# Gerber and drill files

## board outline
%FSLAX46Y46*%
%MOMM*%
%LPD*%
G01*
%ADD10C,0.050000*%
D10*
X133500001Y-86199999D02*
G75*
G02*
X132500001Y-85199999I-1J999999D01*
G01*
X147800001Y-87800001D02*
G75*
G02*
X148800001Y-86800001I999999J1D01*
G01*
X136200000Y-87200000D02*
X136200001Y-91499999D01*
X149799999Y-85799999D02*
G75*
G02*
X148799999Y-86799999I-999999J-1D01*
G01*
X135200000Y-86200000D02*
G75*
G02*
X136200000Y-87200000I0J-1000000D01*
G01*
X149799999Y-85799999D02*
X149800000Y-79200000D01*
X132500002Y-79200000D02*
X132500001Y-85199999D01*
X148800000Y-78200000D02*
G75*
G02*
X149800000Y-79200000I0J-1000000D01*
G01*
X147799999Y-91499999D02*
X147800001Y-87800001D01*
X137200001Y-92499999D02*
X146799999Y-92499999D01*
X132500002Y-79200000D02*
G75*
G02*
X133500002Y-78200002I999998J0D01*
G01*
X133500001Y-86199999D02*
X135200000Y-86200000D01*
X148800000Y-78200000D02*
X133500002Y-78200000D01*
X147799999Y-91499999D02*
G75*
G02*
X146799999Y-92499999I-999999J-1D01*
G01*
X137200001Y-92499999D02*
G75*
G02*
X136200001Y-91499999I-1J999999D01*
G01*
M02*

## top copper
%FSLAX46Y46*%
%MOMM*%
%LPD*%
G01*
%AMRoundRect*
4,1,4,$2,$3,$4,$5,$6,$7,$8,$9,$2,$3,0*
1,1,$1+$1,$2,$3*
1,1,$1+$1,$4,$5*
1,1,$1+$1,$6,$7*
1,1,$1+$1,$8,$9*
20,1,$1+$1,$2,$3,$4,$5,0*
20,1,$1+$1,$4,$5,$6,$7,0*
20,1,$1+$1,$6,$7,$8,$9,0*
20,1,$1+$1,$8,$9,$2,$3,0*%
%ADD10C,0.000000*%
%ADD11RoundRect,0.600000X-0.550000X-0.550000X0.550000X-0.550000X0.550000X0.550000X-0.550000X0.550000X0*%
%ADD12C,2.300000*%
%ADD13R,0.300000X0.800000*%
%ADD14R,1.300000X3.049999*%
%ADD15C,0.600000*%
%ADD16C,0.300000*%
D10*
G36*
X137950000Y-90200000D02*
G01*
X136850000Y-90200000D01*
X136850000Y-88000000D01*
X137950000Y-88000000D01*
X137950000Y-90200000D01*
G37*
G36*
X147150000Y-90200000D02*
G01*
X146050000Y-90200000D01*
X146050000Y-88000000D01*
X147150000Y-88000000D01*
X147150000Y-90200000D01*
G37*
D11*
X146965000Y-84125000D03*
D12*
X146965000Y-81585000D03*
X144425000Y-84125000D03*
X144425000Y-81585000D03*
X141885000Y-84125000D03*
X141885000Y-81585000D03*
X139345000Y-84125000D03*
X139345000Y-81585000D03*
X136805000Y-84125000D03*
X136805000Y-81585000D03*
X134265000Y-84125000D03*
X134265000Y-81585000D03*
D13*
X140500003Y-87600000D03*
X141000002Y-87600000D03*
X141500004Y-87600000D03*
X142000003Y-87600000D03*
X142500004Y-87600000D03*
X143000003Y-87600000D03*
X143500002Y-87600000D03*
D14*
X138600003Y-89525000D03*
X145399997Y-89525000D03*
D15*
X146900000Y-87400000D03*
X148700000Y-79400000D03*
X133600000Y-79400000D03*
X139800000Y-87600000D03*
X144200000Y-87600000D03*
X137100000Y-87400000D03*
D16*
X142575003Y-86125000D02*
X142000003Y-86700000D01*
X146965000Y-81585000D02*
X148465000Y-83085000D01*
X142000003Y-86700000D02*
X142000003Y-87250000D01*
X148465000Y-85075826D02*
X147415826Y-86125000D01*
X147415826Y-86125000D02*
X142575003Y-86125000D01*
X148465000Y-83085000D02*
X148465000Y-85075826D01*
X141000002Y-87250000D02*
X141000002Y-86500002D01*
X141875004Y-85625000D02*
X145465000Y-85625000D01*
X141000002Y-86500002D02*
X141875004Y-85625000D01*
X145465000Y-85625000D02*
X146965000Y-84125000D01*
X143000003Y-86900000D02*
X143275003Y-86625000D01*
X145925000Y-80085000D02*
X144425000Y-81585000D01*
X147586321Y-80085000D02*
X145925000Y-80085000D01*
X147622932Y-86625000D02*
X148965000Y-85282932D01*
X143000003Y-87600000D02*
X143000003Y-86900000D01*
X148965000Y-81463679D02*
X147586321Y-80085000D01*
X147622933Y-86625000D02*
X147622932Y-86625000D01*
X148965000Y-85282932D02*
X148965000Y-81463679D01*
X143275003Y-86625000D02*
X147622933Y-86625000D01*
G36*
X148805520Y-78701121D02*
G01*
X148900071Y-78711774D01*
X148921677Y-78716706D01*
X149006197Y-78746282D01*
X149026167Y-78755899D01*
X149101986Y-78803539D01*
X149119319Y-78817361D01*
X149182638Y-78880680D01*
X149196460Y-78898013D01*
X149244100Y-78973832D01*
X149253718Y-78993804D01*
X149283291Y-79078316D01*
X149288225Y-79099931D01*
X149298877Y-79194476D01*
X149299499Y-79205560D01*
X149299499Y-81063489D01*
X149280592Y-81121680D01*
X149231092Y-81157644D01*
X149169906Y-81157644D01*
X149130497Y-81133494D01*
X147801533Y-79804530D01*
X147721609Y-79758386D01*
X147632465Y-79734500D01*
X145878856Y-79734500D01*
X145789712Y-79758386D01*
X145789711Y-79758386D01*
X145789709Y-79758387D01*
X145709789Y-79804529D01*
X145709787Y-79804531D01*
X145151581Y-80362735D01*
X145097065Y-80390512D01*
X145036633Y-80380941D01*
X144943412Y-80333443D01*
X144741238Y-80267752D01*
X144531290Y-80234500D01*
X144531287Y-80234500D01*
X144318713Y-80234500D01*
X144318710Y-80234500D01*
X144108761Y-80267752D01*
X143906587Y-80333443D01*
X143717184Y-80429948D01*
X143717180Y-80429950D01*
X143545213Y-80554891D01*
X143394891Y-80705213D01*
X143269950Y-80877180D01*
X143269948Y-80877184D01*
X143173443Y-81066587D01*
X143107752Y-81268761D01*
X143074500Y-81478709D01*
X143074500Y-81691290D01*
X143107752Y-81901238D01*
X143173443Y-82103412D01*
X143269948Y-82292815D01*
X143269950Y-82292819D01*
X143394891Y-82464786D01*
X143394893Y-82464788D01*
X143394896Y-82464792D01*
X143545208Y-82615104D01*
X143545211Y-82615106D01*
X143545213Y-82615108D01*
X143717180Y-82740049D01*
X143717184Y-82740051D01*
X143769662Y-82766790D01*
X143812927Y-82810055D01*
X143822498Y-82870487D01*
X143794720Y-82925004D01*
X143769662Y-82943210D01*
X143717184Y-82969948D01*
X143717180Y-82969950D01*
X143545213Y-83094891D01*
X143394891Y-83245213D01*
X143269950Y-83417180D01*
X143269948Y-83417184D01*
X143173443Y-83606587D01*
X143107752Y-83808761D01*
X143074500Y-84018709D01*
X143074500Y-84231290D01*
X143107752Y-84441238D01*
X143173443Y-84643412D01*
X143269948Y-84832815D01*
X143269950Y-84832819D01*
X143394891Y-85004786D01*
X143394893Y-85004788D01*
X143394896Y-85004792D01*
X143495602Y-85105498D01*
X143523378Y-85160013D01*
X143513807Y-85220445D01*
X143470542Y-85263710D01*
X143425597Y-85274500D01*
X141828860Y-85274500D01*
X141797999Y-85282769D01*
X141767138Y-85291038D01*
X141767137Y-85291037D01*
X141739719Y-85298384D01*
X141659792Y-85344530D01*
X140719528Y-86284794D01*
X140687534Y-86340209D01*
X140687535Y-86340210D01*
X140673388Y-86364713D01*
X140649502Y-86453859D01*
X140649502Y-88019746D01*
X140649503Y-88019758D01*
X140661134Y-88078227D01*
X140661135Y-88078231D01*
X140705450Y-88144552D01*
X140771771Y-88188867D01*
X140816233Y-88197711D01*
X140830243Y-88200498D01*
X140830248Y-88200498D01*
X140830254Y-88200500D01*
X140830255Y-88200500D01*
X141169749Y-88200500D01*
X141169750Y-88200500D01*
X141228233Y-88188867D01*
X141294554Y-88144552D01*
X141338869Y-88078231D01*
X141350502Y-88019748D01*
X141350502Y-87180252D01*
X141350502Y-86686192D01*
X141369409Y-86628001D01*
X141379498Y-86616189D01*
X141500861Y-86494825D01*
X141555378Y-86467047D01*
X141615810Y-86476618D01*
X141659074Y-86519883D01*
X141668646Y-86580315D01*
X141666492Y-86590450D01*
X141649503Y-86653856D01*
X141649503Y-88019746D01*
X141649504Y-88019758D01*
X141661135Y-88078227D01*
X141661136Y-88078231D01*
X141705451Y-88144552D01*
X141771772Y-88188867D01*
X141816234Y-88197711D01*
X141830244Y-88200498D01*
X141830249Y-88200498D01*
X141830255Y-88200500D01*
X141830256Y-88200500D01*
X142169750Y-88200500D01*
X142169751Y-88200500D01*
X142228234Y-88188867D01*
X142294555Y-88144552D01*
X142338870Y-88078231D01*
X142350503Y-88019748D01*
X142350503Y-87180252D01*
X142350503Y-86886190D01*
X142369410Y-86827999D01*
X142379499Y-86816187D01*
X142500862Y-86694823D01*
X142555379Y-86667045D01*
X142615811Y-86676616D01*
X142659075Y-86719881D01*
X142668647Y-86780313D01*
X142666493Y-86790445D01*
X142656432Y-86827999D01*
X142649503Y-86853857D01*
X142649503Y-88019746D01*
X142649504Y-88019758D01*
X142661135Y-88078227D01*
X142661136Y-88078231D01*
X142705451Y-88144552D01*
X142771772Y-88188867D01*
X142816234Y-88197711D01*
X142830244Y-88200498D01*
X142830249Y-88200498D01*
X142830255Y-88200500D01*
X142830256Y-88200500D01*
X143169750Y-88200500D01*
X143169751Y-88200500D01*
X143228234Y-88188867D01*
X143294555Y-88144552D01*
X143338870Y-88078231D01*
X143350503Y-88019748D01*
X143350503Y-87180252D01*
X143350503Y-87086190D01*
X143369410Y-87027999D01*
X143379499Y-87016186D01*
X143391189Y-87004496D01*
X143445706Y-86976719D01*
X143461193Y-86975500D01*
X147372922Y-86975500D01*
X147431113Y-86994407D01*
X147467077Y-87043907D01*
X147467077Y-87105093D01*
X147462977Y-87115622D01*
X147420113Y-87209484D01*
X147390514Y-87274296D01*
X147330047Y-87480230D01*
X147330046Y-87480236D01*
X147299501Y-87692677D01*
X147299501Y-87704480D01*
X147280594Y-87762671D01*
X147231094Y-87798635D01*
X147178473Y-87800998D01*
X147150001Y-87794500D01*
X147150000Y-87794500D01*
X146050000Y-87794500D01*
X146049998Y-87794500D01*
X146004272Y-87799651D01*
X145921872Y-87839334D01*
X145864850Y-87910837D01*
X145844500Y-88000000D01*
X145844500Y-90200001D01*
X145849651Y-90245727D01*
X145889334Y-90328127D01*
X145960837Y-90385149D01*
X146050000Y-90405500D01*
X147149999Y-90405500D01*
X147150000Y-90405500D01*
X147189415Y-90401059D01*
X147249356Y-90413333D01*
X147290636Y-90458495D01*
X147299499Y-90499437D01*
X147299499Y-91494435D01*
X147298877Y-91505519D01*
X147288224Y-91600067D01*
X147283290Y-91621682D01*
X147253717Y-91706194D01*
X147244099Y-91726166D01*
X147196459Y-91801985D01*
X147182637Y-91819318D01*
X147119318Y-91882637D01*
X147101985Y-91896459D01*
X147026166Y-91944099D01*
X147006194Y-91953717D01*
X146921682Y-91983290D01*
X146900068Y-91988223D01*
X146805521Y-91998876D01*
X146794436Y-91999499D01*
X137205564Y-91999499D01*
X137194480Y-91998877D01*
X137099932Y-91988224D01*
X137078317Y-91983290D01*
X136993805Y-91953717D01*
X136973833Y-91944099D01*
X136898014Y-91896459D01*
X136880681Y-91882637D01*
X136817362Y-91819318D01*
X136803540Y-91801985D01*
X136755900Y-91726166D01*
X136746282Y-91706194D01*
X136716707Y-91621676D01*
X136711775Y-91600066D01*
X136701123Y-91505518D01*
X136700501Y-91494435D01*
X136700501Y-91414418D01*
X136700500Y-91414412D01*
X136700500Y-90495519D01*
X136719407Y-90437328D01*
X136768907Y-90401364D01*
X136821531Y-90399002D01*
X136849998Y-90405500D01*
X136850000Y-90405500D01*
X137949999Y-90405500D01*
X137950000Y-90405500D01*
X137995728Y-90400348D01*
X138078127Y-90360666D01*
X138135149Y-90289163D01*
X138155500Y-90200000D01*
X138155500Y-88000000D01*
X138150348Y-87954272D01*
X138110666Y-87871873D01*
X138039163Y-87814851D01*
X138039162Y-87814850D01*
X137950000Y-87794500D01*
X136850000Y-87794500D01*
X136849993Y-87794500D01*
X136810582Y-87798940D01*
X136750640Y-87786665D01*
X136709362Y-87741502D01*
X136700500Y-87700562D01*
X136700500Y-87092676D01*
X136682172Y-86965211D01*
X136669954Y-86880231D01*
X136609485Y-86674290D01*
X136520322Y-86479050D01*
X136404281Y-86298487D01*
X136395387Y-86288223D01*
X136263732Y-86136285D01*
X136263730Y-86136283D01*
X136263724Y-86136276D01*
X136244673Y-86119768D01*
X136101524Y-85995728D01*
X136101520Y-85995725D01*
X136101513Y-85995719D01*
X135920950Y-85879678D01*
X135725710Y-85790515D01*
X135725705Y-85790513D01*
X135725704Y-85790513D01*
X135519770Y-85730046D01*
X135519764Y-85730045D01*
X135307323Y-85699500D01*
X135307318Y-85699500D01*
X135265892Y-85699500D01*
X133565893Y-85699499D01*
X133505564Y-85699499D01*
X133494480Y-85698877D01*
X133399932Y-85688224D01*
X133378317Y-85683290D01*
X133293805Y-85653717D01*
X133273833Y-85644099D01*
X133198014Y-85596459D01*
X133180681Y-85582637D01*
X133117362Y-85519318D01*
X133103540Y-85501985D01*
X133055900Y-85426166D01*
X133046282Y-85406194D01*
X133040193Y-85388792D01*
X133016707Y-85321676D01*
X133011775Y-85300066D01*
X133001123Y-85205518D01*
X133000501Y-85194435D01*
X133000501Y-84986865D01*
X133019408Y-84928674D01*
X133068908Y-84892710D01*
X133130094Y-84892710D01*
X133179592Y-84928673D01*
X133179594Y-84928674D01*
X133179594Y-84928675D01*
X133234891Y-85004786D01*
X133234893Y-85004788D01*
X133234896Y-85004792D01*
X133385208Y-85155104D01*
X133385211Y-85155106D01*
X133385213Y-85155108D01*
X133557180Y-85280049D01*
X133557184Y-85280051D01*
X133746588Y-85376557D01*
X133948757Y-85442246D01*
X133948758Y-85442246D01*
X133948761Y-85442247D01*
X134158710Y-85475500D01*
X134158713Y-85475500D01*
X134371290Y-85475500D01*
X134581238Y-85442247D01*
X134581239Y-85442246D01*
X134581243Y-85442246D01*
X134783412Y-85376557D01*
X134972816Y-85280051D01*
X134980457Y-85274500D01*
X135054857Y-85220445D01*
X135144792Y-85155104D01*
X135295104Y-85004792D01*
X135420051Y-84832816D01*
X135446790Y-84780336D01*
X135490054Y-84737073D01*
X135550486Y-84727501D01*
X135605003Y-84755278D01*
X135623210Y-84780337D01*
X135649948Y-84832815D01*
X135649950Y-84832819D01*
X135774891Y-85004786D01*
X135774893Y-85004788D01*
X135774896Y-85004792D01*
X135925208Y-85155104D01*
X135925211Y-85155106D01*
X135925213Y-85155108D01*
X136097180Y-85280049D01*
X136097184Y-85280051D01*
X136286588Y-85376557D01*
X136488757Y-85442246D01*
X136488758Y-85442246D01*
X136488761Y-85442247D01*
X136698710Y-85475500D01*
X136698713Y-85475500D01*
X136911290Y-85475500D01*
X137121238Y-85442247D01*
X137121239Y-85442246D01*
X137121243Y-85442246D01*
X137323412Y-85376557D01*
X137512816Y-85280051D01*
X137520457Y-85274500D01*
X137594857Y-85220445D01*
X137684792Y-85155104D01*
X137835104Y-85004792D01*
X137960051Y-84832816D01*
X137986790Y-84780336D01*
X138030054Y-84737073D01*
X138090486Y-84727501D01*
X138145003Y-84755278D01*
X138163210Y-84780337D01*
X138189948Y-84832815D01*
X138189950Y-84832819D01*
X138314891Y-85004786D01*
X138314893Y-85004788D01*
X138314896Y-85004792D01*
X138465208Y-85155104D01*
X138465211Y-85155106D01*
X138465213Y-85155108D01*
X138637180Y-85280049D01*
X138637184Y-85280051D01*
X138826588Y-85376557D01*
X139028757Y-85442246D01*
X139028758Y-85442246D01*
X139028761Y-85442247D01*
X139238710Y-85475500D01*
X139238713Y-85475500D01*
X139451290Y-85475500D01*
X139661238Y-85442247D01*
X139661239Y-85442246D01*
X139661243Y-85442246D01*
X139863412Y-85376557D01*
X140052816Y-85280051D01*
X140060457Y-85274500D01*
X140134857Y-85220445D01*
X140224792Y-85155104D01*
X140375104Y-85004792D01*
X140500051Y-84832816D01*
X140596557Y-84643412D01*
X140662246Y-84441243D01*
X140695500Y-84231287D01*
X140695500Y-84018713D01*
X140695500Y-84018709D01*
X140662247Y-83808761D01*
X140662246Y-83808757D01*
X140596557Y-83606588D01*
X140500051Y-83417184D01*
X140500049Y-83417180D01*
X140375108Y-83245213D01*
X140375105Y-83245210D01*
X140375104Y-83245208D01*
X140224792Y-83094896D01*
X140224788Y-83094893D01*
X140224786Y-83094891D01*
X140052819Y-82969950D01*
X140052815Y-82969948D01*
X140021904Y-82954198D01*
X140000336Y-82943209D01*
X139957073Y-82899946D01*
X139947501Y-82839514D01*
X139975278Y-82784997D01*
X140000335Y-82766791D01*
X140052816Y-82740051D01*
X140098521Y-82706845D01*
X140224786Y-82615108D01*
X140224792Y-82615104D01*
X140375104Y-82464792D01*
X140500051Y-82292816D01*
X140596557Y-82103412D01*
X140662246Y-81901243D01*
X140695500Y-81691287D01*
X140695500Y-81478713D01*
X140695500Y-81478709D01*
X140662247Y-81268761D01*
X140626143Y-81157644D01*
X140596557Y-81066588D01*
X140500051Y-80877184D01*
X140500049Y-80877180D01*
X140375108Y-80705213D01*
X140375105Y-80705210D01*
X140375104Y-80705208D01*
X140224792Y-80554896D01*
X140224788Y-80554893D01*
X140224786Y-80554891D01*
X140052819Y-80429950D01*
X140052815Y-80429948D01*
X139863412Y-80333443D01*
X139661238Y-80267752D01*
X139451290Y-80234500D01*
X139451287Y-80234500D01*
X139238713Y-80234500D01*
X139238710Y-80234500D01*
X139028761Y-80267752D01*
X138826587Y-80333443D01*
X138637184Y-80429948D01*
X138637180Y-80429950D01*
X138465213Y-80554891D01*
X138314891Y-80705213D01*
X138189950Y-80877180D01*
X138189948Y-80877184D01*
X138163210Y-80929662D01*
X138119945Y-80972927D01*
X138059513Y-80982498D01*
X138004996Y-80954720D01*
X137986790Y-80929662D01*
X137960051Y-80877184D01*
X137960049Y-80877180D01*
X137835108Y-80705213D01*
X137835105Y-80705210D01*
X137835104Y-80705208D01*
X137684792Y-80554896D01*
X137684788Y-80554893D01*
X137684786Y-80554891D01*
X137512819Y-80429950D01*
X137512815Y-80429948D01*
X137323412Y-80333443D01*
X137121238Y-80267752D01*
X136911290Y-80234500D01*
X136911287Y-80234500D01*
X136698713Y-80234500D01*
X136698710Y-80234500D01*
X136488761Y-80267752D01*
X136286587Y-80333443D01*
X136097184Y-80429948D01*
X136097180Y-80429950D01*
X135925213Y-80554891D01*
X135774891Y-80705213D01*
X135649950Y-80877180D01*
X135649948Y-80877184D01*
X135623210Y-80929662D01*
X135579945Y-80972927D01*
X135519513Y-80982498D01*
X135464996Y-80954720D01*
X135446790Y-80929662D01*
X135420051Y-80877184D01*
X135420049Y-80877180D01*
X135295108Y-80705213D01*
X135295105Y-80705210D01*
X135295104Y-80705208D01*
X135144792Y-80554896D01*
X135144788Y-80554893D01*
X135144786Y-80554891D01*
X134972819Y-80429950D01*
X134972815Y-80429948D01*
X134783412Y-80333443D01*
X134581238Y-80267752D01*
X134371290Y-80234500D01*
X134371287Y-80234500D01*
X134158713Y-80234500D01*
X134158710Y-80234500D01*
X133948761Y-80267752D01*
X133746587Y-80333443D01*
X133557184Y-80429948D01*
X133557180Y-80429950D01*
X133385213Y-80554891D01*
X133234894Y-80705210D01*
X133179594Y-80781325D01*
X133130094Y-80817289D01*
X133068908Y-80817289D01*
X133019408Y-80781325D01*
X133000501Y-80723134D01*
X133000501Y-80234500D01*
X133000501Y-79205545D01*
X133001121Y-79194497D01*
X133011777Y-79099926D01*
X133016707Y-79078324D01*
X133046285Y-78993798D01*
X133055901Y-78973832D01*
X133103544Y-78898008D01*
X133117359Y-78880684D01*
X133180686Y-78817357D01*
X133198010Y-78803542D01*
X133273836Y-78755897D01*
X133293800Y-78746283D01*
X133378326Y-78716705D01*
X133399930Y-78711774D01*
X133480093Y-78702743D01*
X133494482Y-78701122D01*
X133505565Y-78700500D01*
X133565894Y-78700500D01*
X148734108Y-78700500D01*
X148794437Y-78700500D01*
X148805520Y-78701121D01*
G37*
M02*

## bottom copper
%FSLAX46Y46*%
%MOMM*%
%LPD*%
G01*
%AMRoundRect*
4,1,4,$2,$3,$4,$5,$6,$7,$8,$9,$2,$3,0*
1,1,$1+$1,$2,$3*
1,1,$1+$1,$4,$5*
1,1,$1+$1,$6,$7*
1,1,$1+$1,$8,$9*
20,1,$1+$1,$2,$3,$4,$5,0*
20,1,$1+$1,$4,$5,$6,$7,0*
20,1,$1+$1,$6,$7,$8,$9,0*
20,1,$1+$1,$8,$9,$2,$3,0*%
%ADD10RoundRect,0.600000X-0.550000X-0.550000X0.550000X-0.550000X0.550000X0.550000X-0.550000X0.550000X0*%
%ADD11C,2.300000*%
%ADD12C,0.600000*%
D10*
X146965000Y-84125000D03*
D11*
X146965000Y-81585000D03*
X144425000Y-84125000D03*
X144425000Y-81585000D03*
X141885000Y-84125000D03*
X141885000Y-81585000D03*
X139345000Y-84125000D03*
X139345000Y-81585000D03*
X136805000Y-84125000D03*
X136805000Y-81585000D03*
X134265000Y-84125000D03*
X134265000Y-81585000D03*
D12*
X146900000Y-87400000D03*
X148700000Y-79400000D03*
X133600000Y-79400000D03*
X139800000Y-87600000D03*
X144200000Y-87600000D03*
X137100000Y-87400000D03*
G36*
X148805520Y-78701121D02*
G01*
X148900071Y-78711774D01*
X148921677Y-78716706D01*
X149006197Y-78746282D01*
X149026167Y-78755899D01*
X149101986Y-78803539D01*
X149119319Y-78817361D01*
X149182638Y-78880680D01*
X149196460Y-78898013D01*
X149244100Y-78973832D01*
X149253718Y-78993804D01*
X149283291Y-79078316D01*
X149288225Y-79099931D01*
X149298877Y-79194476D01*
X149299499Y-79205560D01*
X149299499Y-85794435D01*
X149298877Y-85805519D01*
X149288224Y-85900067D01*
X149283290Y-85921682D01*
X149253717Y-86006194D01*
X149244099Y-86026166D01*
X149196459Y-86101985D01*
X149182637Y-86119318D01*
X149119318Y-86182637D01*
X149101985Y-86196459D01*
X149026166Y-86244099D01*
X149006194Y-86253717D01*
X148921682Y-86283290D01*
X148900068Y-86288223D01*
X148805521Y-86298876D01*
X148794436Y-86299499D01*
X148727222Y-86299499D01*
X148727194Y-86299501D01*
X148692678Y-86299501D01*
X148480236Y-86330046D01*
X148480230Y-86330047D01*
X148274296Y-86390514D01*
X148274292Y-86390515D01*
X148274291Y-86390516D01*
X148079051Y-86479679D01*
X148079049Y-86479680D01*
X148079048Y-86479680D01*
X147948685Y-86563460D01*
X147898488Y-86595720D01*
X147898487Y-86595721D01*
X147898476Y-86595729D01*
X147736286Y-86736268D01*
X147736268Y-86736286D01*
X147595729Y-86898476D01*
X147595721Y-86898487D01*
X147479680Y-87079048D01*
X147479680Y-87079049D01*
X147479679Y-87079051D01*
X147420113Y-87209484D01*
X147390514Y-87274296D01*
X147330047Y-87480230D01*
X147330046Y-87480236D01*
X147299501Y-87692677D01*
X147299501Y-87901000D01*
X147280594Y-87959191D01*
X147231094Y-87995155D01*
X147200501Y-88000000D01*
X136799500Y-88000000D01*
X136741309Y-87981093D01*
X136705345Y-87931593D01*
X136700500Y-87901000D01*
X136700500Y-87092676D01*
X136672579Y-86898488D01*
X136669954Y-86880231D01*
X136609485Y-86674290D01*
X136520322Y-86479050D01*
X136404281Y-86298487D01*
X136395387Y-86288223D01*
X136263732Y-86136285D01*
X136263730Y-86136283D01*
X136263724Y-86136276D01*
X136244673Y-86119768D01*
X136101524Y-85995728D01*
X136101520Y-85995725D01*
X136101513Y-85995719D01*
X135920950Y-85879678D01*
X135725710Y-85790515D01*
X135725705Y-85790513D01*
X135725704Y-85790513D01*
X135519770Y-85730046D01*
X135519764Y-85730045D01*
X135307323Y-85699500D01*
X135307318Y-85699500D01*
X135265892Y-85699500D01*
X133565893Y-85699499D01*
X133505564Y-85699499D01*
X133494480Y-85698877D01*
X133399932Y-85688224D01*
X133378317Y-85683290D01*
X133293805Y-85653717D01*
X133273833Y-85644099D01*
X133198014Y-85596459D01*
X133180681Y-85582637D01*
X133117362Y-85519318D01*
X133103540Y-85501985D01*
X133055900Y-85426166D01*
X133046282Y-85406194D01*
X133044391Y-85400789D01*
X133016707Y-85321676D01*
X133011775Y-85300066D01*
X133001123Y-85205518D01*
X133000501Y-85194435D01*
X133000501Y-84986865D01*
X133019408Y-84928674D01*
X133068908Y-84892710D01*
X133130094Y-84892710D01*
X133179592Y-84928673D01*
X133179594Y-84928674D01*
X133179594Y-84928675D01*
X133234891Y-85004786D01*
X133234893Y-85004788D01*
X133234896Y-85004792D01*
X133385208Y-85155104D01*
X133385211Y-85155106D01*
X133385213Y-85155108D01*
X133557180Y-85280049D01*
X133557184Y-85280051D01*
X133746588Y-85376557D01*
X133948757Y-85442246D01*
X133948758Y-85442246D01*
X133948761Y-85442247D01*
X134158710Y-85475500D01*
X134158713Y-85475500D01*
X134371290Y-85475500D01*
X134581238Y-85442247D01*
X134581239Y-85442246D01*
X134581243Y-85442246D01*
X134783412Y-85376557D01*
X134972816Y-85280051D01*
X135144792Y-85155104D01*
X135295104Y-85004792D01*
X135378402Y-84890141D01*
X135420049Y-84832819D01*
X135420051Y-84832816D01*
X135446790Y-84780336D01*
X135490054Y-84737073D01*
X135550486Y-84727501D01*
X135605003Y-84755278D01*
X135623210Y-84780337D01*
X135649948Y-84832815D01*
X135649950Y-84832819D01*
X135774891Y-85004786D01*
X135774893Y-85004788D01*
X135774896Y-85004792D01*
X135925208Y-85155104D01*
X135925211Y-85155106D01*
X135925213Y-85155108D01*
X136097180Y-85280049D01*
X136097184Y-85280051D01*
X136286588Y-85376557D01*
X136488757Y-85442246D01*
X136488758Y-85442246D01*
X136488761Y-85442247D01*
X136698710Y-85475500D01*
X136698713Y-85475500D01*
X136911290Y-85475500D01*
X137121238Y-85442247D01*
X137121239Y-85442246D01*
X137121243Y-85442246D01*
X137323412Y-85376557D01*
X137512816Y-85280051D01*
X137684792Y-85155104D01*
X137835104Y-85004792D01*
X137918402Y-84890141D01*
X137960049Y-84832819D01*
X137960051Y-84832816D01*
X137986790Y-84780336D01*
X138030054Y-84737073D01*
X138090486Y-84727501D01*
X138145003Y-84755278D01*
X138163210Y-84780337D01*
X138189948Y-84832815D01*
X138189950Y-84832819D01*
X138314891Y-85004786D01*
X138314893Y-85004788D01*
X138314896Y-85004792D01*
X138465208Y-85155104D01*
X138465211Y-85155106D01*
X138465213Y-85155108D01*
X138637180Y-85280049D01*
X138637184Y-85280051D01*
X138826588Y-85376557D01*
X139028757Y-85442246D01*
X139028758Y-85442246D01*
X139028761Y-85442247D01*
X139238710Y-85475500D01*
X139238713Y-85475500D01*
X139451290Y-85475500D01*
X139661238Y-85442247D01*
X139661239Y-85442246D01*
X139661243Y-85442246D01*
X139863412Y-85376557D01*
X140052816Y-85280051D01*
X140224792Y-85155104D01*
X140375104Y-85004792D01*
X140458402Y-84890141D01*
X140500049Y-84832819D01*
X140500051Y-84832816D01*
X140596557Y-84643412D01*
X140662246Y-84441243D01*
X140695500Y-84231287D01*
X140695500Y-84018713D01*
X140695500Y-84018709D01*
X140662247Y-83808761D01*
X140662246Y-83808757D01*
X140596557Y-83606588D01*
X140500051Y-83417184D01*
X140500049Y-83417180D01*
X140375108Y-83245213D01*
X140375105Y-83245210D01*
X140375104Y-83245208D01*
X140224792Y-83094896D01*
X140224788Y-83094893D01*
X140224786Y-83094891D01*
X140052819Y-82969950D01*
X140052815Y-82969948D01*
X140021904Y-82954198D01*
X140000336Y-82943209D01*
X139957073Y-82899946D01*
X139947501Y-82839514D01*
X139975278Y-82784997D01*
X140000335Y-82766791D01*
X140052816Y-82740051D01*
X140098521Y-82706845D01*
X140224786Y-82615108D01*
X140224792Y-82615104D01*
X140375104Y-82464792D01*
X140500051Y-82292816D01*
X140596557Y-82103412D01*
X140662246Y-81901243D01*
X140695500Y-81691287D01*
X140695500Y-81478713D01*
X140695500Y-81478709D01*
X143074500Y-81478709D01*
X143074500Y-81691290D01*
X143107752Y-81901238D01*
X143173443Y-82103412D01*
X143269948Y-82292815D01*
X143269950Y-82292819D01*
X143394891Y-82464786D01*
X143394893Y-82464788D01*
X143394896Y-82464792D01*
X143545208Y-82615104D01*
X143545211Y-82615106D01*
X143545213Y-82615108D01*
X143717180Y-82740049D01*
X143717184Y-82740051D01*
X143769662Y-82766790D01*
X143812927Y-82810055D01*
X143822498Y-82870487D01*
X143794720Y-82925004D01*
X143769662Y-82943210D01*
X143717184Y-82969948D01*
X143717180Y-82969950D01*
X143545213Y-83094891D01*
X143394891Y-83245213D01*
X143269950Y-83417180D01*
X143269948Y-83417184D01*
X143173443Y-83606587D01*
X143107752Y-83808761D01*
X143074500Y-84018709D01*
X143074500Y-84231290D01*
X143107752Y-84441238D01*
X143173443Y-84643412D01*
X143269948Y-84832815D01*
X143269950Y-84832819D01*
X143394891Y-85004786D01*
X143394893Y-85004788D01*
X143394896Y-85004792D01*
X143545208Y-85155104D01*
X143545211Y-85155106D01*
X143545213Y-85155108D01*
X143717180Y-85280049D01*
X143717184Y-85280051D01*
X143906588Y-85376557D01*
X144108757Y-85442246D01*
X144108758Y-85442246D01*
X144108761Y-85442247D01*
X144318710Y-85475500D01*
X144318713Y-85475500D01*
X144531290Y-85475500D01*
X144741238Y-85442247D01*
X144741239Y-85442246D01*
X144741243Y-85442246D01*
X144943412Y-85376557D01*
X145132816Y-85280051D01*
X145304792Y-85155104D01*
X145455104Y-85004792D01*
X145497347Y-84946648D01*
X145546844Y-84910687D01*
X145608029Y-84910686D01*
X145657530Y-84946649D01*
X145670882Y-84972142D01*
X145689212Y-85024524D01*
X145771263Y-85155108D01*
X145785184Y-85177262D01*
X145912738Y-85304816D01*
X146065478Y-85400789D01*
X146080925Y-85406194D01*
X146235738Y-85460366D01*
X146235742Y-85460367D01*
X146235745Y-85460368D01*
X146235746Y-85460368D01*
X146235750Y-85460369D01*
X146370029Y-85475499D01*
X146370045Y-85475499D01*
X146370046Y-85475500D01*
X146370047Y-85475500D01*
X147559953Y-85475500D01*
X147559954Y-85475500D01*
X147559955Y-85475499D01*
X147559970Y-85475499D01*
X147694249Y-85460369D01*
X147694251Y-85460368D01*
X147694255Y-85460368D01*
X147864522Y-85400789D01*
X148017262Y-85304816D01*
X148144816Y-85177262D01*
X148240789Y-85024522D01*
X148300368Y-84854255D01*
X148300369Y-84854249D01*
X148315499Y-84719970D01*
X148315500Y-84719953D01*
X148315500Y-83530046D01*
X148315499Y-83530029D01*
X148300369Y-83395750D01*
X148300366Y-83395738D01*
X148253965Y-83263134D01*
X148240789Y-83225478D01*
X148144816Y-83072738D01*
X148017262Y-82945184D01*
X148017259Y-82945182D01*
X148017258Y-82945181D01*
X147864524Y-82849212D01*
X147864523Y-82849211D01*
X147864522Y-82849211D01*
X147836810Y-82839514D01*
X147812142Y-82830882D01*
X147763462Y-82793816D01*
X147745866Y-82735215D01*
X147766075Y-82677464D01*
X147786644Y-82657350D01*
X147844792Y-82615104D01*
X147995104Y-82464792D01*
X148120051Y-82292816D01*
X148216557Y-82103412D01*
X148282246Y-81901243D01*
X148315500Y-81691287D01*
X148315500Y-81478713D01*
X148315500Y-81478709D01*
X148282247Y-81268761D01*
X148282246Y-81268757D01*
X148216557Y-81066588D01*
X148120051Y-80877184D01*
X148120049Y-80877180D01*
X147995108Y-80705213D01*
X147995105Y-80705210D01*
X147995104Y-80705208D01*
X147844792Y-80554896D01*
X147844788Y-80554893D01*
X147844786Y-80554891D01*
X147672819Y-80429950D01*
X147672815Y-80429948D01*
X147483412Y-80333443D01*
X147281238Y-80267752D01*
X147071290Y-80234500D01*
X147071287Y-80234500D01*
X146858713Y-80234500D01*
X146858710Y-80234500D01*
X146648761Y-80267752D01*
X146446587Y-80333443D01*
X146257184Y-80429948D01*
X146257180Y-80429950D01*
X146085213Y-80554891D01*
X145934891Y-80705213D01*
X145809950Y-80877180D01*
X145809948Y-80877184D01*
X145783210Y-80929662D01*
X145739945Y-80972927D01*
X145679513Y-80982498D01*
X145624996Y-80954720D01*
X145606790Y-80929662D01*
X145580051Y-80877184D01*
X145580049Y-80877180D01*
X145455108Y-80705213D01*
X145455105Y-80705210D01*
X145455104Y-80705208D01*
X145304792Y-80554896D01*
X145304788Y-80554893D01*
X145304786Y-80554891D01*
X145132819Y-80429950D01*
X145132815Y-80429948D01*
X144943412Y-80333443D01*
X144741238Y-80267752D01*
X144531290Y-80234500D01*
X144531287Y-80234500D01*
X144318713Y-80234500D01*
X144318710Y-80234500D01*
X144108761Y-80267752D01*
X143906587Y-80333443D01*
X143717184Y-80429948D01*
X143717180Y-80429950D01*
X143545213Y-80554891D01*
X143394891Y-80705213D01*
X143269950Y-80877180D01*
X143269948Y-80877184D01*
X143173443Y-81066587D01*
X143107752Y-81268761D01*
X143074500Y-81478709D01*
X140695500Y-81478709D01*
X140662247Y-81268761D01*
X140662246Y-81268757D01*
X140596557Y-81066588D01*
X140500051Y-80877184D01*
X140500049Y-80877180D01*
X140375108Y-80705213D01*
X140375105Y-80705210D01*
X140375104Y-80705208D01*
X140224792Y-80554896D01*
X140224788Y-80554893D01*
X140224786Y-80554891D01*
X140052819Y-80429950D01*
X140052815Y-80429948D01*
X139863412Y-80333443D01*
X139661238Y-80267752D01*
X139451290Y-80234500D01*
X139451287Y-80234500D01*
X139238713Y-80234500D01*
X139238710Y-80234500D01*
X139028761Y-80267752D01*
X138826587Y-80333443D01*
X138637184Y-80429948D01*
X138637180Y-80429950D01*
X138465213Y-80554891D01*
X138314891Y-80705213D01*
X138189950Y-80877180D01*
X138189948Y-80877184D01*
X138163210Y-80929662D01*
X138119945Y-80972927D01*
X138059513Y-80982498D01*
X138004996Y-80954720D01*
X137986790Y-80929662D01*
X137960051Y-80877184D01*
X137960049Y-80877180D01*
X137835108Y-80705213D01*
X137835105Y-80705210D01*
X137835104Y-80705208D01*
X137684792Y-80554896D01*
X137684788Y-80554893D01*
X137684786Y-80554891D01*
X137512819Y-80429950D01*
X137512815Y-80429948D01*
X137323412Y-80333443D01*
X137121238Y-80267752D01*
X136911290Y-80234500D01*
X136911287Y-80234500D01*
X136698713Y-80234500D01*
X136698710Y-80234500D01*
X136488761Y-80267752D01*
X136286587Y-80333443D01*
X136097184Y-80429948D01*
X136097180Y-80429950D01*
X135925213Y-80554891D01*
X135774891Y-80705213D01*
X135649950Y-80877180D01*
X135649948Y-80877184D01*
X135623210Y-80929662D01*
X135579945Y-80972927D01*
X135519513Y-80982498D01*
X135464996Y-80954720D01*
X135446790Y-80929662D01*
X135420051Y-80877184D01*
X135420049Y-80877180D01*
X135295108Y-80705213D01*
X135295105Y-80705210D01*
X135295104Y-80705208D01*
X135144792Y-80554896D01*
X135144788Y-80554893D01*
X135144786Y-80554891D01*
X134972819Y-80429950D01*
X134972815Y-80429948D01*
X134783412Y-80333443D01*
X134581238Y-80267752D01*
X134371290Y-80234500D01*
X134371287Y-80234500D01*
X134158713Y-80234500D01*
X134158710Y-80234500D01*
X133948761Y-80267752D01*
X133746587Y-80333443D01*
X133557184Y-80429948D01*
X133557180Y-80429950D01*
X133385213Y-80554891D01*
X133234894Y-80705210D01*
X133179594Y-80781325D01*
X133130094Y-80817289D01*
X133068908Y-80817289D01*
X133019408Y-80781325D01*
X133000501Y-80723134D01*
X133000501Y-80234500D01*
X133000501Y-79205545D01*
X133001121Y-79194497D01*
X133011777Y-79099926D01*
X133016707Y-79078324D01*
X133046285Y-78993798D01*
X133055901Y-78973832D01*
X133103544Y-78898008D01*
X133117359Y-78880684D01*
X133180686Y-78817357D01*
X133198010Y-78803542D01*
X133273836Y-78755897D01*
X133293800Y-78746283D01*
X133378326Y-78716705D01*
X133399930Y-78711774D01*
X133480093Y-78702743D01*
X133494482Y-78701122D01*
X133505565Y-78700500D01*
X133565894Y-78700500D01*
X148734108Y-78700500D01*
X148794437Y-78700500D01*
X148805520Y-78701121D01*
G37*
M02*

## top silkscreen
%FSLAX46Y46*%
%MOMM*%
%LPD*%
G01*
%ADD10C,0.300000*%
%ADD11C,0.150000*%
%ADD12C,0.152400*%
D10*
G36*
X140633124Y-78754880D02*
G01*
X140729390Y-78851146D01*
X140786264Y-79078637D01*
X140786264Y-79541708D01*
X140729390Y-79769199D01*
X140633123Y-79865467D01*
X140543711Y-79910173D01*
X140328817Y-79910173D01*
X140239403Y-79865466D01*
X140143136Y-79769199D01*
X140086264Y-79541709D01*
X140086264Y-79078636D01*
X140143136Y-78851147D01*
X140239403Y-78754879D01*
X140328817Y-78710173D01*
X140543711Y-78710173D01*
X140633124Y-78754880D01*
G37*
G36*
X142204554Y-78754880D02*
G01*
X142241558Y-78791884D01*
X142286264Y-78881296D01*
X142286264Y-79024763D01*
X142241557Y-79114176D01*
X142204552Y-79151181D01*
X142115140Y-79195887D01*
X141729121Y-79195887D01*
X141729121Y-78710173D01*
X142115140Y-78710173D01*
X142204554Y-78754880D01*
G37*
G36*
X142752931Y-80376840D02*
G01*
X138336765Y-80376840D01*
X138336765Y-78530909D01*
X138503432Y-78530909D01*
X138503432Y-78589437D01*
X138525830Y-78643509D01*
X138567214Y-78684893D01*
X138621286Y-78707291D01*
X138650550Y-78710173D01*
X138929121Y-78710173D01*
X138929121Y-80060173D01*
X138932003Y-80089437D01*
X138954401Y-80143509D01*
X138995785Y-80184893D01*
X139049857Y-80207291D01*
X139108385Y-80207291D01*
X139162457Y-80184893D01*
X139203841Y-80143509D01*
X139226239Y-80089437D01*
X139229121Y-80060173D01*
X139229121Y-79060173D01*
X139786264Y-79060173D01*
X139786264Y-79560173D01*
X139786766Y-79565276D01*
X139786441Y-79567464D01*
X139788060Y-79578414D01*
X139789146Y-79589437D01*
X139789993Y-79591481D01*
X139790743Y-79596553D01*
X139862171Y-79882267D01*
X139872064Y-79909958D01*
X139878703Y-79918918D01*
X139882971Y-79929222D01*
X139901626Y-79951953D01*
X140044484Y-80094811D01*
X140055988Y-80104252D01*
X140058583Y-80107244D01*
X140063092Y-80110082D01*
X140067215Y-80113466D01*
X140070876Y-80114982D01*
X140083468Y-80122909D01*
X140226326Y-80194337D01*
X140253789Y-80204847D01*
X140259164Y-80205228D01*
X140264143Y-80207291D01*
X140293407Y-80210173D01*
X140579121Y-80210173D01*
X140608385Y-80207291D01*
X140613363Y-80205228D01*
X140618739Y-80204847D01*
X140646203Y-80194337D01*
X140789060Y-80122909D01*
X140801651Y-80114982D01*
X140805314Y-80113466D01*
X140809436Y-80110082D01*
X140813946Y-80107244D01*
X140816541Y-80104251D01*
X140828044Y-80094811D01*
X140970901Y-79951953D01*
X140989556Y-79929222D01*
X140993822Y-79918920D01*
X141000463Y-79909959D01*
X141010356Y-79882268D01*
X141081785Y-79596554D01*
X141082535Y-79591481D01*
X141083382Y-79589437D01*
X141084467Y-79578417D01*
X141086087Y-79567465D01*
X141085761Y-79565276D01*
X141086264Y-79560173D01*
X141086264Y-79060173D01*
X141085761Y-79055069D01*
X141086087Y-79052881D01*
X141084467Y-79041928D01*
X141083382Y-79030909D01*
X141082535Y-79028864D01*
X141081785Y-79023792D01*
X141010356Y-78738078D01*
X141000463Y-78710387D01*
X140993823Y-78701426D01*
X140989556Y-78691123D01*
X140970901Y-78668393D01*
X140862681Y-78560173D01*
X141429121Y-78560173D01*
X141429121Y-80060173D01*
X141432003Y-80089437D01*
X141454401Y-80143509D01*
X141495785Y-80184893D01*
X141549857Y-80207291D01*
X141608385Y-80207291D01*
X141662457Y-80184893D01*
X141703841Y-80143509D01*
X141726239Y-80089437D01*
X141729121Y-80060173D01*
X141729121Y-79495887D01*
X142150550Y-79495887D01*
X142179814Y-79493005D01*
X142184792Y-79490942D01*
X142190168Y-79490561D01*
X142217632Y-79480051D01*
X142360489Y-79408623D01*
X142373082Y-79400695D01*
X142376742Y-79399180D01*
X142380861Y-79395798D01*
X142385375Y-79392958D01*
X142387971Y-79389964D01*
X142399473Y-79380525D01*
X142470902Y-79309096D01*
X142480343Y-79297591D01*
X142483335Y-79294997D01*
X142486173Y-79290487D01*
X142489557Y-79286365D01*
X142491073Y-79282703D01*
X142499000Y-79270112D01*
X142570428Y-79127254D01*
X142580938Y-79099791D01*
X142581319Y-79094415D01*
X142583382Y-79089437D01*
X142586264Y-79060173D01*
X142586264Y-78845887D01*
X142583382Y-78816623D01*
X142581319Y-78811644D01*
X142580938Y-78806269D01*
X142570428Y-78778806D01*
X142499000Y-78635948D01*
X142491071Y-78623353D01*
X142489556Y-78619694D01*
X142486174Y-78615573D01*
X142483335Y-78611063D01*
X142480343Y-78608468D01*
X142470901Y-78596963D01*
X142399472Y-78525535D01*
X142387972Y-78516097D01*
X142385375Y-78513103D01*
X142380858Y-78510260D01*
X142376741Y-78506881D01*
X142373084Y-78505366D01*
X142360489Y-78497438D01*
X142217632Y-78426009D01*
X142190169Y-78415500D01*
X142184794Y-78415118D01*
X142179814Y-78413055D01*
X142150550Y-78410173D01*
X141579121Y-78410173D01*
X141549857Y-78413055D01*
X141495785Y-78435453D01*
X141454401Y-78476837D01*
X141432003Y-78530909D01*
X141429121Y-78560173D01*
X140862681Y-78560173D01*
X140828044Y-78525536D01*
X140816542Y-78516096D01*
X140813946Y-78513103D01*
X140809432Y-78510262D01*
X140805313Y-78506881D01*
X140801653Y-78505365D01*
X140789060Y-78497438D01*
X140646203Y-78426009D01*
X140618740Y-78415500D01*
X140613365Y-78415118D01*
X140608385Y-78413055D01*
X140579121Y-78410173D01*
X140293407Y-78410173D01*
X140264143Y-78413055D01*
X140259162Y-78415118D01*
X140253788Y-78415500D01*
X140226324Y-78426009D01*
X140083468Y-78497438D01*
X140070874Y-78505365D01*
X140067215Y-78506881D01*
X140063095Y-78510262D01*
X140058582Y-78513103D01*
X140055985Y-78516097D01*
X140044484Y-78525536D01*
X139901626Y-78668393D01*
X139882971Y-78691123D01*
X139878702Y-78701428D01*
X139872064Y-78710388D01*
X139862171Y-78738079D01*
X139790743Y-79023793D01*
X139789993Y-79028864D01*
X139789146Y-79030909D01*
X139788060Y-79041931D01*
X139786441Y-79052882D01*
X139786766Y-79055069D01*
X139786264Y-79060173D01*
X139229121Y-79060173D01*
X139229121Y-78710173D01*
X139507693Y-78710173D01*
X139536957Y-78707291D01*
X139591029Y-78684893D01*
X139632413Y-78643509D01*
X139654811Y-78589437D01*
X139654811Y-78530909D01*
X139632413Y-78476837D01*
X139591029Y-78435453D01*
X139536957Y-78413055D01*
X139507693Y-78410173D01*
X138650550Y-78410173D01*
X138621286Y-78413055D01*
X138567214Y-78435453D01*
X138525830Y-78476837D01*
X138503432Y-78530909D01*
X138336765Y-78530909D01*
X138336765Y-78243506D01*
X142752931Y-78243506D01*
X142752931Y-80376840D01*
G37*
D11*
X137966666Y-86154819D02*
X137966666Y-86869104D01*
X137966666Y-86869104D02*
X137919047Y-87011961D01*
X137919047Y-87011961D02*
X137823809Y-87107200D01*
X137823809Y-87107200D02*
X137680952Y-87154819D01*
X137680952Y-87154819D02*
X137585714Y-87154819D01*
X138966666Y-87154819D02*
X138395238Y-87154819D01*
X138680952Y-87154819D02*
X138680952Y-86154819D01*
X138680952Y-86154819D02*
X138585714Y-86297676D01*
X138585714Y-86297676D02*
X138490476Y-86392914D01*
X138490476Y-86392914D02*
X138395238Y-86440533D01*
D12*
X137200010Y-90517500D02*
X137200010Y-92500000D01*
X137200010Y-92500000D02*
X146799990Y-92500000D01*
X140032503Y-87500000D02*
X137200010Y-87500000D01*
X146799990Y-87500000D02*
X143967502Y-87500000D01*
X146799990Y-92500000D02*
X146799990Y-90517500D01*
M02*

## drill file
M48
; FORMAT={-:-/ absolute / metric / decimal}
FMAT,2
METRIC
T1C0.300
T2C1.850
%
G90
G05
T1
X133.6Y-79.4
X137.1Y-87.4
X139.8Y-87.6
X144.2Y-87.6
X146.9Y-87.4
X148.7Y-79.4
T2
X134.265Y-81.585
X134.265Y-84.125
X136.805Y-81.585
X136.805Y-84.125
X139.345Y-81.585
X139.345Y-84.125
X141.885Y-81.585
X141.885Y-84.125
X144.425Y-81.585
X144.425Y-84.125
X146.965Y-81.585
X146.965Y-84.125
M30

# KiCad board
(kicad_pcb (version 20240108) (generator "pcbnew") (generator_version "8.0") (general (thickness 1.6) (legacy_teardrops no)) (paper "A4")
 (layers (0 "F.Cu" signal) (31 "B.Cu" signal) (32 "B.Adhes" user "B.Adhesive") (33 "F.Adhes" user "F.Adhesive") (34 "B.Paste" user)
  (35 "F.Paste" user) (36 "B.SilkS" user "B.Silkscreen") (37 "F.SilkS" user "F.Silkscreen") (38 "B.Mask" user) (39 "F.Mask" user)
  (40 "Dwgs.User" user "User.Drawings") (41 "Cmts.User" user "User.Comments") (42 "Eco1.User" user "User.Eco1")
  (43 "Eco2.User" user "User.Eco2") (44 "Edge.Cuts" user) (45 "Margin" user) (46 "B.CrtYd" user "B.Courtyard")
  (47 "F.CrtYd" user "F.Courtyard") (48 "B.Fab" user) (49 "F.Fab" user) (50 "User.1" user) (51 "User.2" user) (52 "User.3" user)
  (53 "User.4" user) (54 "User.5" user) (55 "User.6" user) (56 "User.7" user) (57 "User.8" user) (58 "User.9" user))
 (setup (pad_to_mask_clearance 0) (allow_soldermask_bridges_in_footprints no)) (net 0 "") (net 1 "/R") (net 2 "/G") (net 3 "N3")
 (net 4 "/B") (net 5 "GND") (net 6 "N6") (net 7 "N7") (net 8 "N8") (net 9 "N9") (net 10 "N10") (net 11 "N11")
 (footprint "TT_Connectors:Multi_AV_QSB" (layer "F.Cu") (at 146.965 84.125)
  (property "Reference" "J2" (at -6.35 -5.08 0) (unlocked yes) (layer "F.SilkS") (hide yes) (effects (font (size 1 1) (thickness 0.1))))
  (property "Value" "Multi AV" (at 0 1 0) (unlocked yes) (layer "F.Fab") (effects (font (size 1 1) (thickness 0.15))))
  (pad "1" thru_hole roundrect (at 0 0) (size 2.3 2.3) (drill 1.85) (layers "*.Cu" "*.Mask") (remove_unused_layers no)
   (roundrect_rratio 0.2608695652) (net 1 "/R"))
  (pad "2" thru_hole circle (at 0 -2.54) (size 2.3 2.3) (drill 1.85) (layers "*.Cu" "*.Mask") (remove_unused_layers no) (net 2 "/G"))
  (pad "3" thru_hole circle (at -2.54 0) (size 2.3 2.3) (drill 1.85) (layers "*.Cu" "*.Mask") (remove_unused_layers no) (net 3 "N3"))
  (pad "4" thru_hole circle (at -2.54 -2.54) (size 2.3 2.3) (drill 1.85) (layers "*.Cu" "*.Mask") (remove_unused_layers no) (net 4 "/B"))
  (pad "5" thru_hole circle (at -5.08 0) (size 2.3 2.3) (drill 1.85) (layers "*.Cu" "*.Mask") (remove_unused_layers no) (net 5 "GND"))
  (pad "6" thru_hole circle (at -5.08 -2.54) (size 2.3 2.3) (drill 1.85) (layers "*.Cu" "*.Mask") (remove_unused_layers no) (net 5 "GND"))
  (pad "7" thru_hole circle (at -7.62 0) (size 2.3 2.3) (drill 1.85) (layers "*.Cu" "*.Mask") (remove_unused_layers no) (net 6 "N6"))
  (pad "8" thru_hole circle (at -7.62 -2.54) (size 2.3 2.3) (drill 1.85) (layers "*.Cu" "*.Mask") (remove_unused_layers no) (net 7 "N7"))
  (pad "9" thru_hole circle (at -10.16 0) (size 2.3 2.3) (drill 1.85) (layers "*.Cu" "*.Mask") (remove_unused_layers no) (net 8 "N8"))
  (pad "10" thru_hole circle (at -10.16 -2.54) (size 2.3 2.3) (drill 1.85) (layers "*.Cu" "*.Mask") (remove_unused_layers no) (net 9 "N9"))
  (pad "11" thru_hole circle (at -12.7 0) (size 2.3 2.3) (drill 1.85) (layers "*.Cu" "*.Mask") (remove_unused_layers no) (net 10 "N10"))
  (pad "12" thru_hole circle (at -12.7 -2.54) (size 2.3 2.3) (drill 1.85) (layers "*.Cu" "*.Mask") (remove_unused_layers no) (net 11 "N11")))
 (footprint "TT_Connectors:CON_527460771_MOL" (layer "F.Cu") (at 142 90)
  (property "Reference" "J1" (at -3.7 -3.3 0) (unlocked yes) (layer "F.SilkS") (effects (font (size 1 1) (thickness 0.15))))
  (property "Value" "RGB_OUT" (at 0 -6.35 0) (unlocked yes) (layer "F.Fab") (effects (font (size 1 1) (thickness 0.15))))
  (fp_poly (pts (xy -4.05 -2) (xy -5.15 -2) (xy -5.15 0.2) (xy -4.05 0.2)) (stroke (width 0) (type solid)) (fill solid) (layer "F.Cu"))
  (fp_poly (pts (xy 4.05 -2) (xy 5.15 -2) (xy 5.15 0.2) (xy 4.05 0.2)) (stroke (width 0) (type solid)) (fill solid) (layer "F.Cu"))
  (fp_line (start -4.79999 0.5175) (end -4.79999 2.5) (stroke (width 0.1524) (type solid)) (layer "F.SilkS"))
  (fp_line (start -4.79999 2.5) (end 4.79999 2.5) (stroke (width 0.1524) (type solid)) (layer "F.SilkS"))
  (fp_line (start -1.967497 -2.5) (end -4.79999 -2.5) (stroke (width 0.1524) (type solid)) (layer "F.SilkS"))
  (fp_line (start 4.79999 -2.5) (end 1.967502 -2.5) (stroke (width 0.1524) (type solid)) (layer "F.SilkS"))
  (fp_line (start 4.79999 2.5) (end 4.79999 0.5175) (stroke (width 0.1524) (type solid)) (layer "F.SilkS"))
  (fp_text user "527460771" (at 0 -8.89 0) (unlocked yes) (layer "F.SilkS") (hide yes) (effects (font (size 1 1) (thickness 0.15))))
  (pad "1" smd rect (at -1.499997 -2.4) (size 0.3 0.8) (layers "F.Cu" "F.Paste" "F.Mask") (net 5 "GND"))
  (pad "2" smd rect (at -0.999998 -2.4) (size 0.3 0.8) (layers "F.Cu" "F.Paste" "F.Mask") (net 1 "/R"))
  (pad "3" smd rect (at -0.499996 -2.4) (size 0.3 0.8) (layers "F.Cu" "F.Paste" "F.Mask") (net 5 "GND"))
  (pad "4" smd rect (at 0.000003 -2.4) (size 0.3 0.8) (layers "F.Cu" "F.Paste" "F.Mask") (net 2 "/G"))
  (pad "5" smd rect (at 0.500004 -2.4) (size 0.3 0.8) (layers "F.Cu" "F.Paste" "F.Mask") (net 5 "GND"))
  (pad "6" smd rect (at 1.000003 -2.4) (size 0.3 0.8) (layers "F.Cu" "F.Paste" "F.Mask") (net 4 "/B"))
  (pad "7" smd rect (at 1.500002 -2.4) (size 0.3 0.8) (layers "F.Cu" "F.Paste" "F.Mask") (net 5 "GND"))
  (pad "MP" smd rect (at -3.399997 -0.475) (size 1.3 3.049999) (layers "F.Cu" "F.Paste" "F.Mask") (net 5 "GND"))
  (pad "MP" smd rect (at 3.399997 -0.475) (size 1.3 3.049999) (layers "F.Cu" "F.Paste" "F.Mask") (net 5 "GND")))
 (gr_arc (start 133.500001 86.199999) (mid 132.792894 85.907106) (end 132.500001 85.199999) (stroke (width 0.05) (type default))
  (layer "Edge.Cuts"))
 (gr_arc (start 147.800001 87.800001) (mid 148.092894 87.092894) (end 148.800001 86.800001) (stroke (width 0.05) (type default))
  (layer "Edge.Cuts"))
 (gr_line (start 136.2 87.2) (end 136.200001 91.499999) (stroke (width 0.05) (type default)) (layer "Edge.Cuts"))
 (gr_arc (start 149.799999 85.799999) (mid 149.507106 86.507106) (end 148.799999 86.799999) (stroke (width 0.05) (type default))
  (layer "Edge.Cuts"))
 (gr_arc (start 135.2 86.2) (mid 135.907107 86.492893) (end 136.2 87.2) (stroke (width 0.05) (type default)) (layer "Edge.Cuts"))
 (gr_line (start 149.799999 85.799999) (end 149.8 79.2) (stroke (width 0.05) (type default)) (layer "Edge.Cuts"))
 (gr_line (start 132.500002 79.2) (end 132.500001 85.199999) (stroke (width 0.05) (type default)) (layer "Edge.Cuts"))
 (gr_arc (start 148.8 78.2) (mid 149.507107 78.492893) (end 149.8 79.2) (stroke (width 0.05) (type default)) (layer "Edge.Cuts"))
 (gr_line (start 147.799999 91.499999) (end 147.800001 87.800001) (stroke (width 0.05) (type default)) (layer "Edge.Cuts"))
 (gr_line (start 137.200001 92.499999) (end 146.799999 92.499999) (stroke (width 0.05) (type default)) (layer "Edge.Cuts"))
 (gr_arc (start 132.500002 79.2) (mid 132.792895 78.492893) (end 133.500002 78.2) (stroke (width 0.05) (type default)) (layer "Edge.Cuts"))
 (gr_line (start 133.500001 86.199999) (end 135.2 86.2) (stroke (width 0.05) (type default)) (layer "Edge.Cuts"))
 (gr_line (start 148.8 78.2) (end 133.500002 78.2) (stroke (width 0.05) (type default)) (layer "Edge.Cuts"))
 (gr_arc (start 147.799999 91.499999) (mid 147.507106 92.207106) (end 146.799999 92.499999) (stroke (width 0.05) (type default))
  (layer "Edge.Cuts"))
 (gr_arc (start 137.200001 92.499999) (mid 136.492894 92.207106) (end 136.200001 91.499999) (stroke (width 0.05) (type default))
  (layer "Edge.Cuts"))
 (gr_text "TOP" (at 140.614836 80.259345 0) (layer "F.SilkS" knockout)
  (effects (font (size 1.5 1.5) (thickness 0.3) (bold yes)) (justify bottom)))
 (segment (start 142.575003 86.125) (end 142.000003 86.7) (width 0.3) (layer "F.Cu") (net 2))
 (segment (start 146.965 81.585) (end 148.465 83.085) (width 0.3) (layer "F.Cu") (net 2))
 (segment (start 142.000003 86.7) (end 142.000003 87.25) (width 0.3) (layer "F.Cu") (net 2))
 (segment (start 148.465 85.075826) (end 147.415826 86.125) (width 0.3) (layer "F.Cu") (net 2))
 (segment (start 147.415826 86.125) (end 142.575003 86.125) (width 0.3) (layer "F.Cu") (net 2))
 (segment (start 148.465 83.085) (end 148.465 85.075826) (width 0.3) (layer "F.Cu") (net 2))
 (segment (start 141.000002 87.25) (end 141.000002 86.500002) (width 0.3) (layer "F.Cu") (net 1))
 (segment (start 141.875004 85.625) (end 145.465 85.625) (width 0.3) (layer "F.Cu") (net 1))
 (segment (start 141.000002 86.500002) (end 141.875004 85.625) (width 0.3) (layer "F.Cu") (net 1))
 (segment (start 145.465 85.625) (end 146.965 84.125) (width 0.3) (layer "F.Cu") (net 1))
 (via (at 146.9 87.4) (size 0.6) (drill 0.3) (layers "F.Cu" "B.Cu") (free yes) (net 5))
 (via (at 148.7 79.4) (size 0.6) (drill 0.3) (layers "F.Cu" "B.Cu") (free yes) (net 5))
 (via (at 133.6 79.4) (size 0.6) (drill 0.3) (layers "F.Cu" "B.Cu") (free yes) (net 5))
 (via (at 139.8 87.6) (size 0.6) (drill 0.3) (layers "F.Cu" "B.Cu") (free yes) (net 5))
 (via (at 144.2 87.6) (size 0.6) (drill 0.3) (layers "F.Cu" "B.Cu") (free yes) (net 5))
 (via (at 137.1 87.4) (size 0.6) (drill 0.3) (layers "F.Cu" "B.Cu") (free yes) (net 5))
 (segment (start 143.000003 86.9) (end 143.275003 86.625) (width 0.3) (layer "F.Cu") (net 4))
 (segment (start 145.925 80.085) (end 144.425 81.585) (width 0.3) (layer "F.Cu") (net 4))
 (segment (start 147.586321 80.085) (end 145.925 80.085) (width 0.3) (layer "F.Cu") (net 4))
 (segment (start 147.622932 86.625) (end 148.965 85.282932) (width 0.3) (layer "F.Cu") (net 4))
 (segment (start 143.000003 87.6) (end 143.000003 86.9) (width 0.3) (layer "F.Cu") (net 4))
 (segment (start 148.965 81.463679) (end 147.586321 80.085) (width 0.3) (layer "F.Cu") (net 4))
 (segment (start 147.622933 86.625) (end 147.622932 86.625) (width 0.3) (layer "F.Cu") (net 4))
 (segment (start 148.965 85.282932) (end 148.965 81.463679) (width 0.3) (layer "F.Cu") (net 4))
 (segment (start 143.275003 86.625) (end 147.622933 86.625) (width 0.3) (layer "F.Cu") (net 4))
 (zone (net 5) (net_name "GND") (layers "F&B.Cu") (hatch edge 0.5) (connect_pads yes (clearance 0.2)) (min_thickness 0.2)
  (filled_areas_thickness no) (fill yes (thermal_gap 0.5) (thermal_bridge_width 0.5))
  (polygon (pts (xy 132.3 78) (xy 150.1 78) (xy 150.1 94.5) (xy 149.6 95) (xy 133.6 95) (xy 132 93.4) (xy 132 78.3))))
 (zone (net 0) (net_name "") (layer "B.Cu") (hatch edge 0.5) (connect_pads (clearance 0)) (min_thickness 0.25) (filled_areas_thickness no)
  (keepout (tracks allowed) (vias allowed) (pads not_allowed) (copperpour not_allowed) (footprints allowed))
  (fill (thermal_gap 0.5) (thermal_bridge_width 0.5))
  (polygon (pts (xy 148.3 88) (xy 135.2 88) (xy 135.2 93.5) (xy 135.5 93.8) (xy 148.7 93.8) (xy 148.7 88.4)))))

